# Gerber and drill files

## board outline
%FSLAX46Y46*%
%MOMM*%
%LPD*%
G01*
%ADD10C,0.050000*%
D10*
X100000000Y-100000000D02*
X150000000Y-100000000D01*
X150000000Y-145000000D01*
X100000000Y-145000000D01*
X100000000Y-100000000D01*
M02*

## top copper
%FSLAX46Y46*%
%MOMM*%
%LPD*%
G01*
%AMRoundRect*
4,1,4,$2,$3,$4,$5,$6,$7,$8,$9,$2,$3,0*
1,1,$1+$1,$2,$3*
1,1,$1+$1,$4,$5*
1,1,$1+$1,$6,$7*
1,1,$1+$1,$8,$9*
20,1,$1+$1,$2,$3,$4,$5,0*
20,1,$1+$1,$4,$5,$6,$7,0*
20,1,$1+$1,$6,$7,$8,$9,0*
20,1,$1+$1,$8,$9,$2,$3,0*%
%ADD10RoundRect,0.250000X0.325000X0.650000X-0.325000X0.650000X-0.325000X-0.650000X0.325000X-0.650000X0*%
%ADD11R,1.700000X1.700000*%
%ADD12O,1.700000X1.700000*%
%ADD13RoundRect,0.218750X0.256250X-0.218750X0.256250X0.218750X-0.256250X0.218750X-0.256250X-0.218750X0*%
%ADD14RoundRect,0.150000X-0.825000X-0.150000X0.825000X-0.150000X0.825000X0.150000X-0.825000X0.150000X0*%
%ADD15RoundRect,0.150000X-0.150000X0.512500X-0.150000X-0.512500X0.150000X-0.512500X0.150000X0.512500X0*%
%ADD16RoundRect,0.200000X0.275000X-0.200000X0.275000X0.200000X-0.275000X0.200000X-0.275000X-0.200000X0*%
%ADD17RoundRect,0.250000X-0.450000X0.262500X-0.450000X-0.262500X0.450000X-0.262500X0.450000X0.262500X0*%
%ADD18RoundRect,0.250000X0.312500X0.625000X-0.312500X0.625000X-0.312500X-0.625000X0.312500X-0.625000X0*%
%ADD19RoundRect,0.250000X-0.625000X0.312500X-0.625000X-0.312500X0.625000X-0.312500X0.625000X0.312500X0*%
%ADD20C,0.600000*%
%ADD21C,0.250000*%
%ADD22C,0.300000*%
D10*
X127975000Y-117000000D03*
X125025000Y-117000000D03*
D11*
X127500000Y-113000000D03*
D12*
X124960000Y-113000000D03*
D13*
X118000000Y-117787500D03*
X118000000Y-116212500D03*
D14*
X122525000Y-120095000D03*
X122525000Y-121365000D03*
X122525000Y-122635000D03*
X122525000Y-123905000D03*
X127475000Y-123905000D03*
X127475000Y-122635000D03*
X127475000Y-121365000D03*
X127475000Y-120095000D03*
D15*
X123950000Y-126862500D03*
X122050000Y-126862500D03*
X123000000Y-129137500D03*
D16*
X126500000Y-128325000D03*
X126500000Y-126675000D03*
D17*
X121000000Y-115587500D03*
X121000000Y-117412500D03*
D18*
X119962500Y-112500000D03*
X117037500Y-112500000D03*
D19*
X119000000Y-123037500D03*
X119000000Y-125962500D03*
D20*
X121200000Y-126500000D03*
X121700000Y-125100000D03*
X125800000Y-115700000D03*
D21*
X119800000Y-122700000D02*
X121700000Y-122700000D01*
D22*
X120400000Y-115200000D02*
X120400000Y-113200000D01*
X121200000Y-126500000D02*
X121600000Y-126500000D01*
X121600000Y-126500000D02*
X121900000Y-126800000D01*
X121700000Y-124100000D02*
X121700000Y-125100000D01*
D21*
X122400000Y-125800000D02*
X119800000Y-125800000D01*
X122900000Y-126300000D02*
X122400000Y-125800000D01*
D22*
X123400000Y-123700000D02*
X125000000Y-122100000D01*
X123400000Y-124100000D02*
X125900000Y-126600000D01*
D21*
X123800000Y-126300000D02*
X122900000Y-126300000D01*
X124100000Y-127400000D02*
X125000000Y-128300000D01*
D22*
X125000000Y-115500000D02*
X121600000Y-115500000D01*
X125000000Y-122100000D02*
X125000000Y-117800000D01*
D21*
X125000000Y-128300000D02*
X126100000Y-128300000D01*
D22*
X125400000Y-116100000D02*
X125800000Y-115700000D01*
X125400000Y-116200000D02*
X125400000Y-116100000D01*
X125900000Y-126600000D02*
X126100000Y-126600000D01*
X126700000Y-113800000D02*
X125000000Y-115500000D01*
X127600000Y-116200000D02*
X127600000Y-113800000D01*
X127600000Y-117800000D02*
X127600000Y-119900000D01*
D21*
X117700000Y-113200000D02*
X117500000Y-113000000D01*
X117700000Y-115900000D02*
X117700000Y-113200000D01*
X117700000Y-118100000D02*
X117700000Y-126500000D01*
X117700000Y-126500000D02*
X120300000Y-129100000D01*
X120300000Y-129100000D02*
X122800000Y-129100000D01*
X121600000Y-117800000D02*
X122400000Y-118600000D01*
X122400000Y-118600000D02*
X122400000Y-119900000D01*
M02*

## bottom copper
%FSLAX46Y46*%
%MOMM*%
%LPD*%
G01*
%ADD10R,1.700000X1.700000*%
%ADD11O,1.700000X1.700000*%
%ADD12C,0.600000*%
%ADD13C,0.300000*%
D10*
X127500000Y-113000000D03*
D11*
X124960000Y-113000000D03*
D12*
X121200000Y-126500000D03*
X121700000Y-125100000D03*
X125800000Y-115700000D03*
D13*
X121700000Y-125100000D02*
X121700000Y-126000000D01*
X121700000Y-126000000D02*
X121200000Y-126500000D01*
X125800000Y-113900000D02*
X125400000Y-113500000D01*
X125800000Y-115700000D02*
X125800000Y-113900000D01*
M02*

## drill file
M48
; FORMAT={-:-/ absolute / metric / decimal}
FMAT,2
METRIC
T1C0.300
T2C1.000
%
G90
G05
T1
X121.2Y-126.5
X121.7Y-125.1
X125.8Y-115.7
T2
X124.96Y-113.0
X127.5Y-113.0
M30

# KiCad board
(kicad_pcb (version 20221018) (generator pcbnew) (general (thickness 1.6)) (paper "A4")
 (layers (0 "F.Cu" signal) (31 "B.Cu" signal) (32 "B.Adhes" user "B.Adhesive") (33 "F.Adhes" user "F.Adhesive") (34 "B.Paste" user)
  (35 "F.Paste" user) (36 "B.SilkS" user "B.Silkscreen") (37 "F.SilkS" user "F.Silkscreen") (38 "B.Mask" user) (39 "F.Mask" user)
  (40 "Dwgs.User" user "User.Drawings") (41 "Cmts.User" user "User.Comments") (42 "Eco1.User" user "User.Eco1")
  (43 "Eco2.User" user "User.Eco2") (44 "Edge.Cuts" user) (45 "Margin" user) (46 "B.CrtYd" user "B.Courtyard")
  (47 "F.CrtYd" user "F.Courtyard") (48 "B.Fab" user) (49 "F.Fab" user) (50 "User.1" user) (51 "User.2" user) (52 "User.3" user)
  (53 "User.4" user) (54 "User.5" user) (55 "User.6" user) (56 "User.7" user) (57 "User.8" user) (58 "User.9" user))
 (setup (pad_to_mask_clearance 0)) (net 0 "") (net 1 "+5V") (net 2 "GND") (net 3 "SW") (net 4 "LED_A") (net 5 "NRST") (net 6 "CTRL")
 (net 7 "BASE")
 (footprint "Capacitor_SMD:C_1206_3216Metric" (layer "F.Cu") (at 126.5 117 180)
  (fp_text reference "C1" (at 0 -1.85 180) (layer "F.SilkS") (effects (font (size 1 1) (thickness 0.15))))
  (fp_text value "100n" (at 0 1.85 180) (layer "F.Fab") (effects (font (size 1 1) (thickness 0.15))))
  (pad "1" smd roundrect (at -1.475 0 180) (size 1.15 1.8) (layers "F.Cu" "F.Paste" "F.Mask") (roundrect_rratio 0.217391) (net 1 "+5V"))
  (pad "2" smd roundrect (at 1.475 0 180) (size 1.15 1.8) (layers "F.Cu" "F.Paste" "F.Mask") (roundrect_rratio 0.217391) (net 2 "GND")))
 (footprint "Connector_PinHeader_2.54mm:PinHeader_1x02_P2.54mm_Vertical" (layer "F.Cu") (at 127.5 113 -90)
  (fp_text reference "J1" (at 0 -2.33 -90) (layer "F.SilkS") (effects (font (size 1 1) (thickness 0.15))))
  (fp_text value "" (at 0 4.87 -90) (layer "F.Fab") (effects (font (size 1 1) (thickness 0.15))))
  (pad "1" thru_hole rect (at 0 0 270) (size 1.7 1.7) (drill 1) (layers "*.Cu" "*.Mask") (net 1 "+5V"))
  (pad "2" thru_hole oval (at 0 2.54 270) (size 1.7 1.7) (drill 1) (layers "*.Cu" "*.Mask") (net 2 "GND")))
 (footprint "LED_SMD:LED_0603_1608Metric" (layer "F.Cu") (at 118 117 90)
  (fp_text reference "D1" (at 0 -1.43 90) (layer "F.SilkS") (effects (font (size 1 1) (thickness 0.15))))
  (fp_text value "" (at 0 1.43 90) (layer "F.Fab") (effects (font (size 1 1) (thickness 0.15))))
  (pad "1" smd roundrect (at -0.7875 0 90) (size 0.875 0.95) (layers "F.Cu" "F.Paste" "F.Mask") (roundrect_rratio 0.25) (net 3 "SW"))
  (pad "2" smd roundrect (at 0.7875 0 90) (size 0.875 0.95) (layers "F.Cu" "F.Paste" "F.Mask") (roundrect_rratio 0.25) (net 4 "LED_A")))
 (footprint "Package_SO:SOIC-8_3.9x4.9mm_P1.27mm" (layer "F.Cu") (at 125 122)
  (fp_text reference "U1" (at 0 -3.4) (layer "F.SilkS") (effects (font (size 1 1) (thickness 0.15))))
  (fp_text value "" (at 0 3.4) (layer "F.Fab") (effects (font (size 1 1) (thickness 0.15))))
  (pad "1" smd roundrect (at -2.475 -1.905) (size 1.95 0.6) (layers "F.Cu" "F.Paste" "F.Mask") (roundrect_rratio 0.25) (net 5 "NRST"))
  (pad "2" smd roundrect (at -2.475 -0.635) (size 1.95 0.6) (layers "F.Cu" "F.Paste" "F.Mask") (roundrect_rratio 0.25))
  (pad "3" smd roundrect (at -2.475 0.635) (size 1.95 0.6) (layers "F.Cu" "F.Paste" "F.Mask") (roundrect_rratio 0.25) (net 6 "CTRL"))
  (pad "4" smd roundrect (at -2.475 1.905) (size 1.95 0.6) (layers "F.Cu" "F.Paste" "F.Mask") (roundrect_rratio 0.25) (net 2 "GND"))
  (pad "5" smd roundrect (at 2.475 1.905) (size 1.95 0.6) (layers "F.Cu" "F.Paste" "F.Mask") (roundrect_rratio 0.25))
  (pad "6" smd roundrect (at 2.475 0.635) (size 1.95 0.6) (layers "F.Cu" "F.Paste" "F.Mask") (roundrect_rratio 0.25))
  (pad "7" smd roundrect (at 2.475 -0.635) (size 1.95 0.6) (layers "F.Cu" "F.Paste" "F.Mask") (roundrect_rratio 0.25))
  (pad "8" smd roundrect (at 2.475 -1.905) (size 1.95 0.6) (layers "F.Cu" "F.Paste" "F.Mask") (roundrect_rratio 0.25) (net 1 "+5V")))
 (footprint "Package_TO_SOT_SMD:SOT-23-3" (layer "F.Cu") (at 123 128 -90)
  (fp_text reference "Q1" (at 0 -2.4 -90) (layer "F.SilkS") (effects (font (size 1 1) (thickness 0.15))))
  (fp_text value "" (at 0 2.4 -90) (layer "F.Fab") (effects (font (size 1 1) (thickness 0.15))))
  (pad "1" smd roundrect (at -1.1375 -0.95 270) (size 1.325 0.6) (layers "F.Cu" "F.Paste" "F.Mask") (roundrect_rratio 0.25) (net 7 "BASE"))
  (pad "2" smd roundrect (at -1.1375 0.95 270) (size 1.325 0.6) (layers "F.Cu" "F.Paste" "F.Mask") (roundrect_rratio 0.25) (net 2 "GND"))
  (pad "3" smd roundrect (at 1.1375 0 270) (size 1.325 0.6) (layers "F.Cu" "F.Paste" "F.Mask") (roundrect_rratio 0.25) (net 3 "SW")))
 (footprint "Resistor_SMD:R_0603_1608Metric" (layer "F.Cu") (at 126.5 127.5 90)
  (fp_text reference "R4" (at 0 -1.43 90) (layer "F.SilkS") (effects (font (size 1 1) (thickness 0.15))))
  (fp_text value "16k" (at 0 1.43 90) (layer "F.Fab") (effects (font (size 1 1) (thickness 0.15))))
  (pad "1" smd roundrect (at -0.825 0 90) (size 0.8 0.95) (layers "F.Cu" "F.Paste" "F.Mask") (roundrect_rratio 0.25) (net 7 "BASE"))
  (pad "2" smd roundrect (at 0.825 0 90) (size 0.8 0.95) (layers "F.Cu" "F.Paste" "F.Mask") (roundrect_rratio 0.25) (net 2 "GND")))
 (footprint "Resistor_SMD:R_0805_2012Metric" (layer "F.Cu") (at 121 116.5 -90)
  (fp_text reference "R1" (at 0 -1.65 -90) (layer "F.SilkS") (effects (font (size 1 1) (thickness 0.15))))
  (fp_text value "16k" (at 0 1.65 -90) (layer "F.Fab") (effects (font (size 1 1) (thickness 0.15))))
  (pad "1" smd roundrect (at -0.9125 0 270) (size 1.025 1.4) (layers "F.Cu" "F.Paste" "F.Mask") (roundrect_rratio 0.243902) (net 1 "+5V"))
  (pad "2" smd roundrect (at 0.9125 0 270) (size 1.025 1.4) (layers "F.Cu" "F.Paste" "F.Mask") (roundrect_rratio 0.243902) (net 5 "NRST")))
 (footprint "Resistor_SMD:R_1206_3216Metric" (layer "F.Cu") (at 118.5 112.5 180)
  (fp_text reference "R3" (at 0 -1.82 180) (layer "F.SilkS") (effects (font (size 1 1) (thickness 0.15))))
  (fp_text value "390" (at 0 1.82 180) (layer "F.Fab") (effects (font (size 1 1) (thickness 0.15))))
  (pad "1" smd roundrect (at -1.4625 0 180) (size 1.125 1.75) (layers "F.Cu" "F.Paste" "F.Mask") (roundrect_rratio 0.222222) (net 1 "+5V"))
  (pad "2" smd roundrect (at 1.4625 0 180) (size 1.125 1.75) (layers "F.Cu" "F.Paste" "F.Mask") (roundrect_rratio 0.222222) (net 4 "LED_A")))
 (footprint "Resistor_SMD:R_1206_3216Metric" (layer "F.Cu") (at 119 124.5 -90)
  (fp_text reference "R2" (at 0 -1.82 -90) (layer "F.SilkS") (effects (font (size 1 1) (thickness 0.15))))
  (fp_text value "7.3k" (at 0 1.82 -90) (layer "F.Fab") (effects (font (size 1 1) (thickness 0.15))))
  (pad "1" smd roundrect (at -1.4625 0 270) (size 1.125 1.75) (layers "F.Cu" "F.Paste" "F.Mask") (roundrect_rratio 0.222222) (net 6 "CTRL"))
  (pad "2" smd roundrect (at 1.4625 0 270) (size 1.125 1.75) (layers "F.Cu" "F.Paste" "F.Mask") (roundrect_rratio 0.222222) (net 7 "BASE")))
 (gr_rect (start 100 100) (end 150 145) (stroke (width 0.05) (type default)) (fill none) (layer "Edge.Cuts"))
 (segment (start 119.8 122.7) (end 121.7 122.7) (width 0.25) (layer "F.Cu") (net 6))
 (segment (start 120.4 115.2) (end 120.4 113.2) (width 0.3) (layer "F.Cu") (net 1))
 (segment (start 121.2 126.5) (end 121.6 126.5) (width 0.3) (layer "F.Cu") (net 2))
 (segment (start 121.6 126.5) (end 121.9 126.8) (width 0.3) (layer "F.Cu") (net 2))
 (segment (start 121.7 124.1) (end 121.7 125.1) (width 0.3) (layer "F.Cu") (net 2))
 (segment (start 122.4 125.8) (end 119.8 125.8) (width 0.25) (layer "F.Cu") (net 7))
 (segment (start 122.9 126.3) (end 122.4 125.8) (width 0.25) (layer "F.Cu") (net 7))
 (segment (start 123.4 123.7) (end 125 122.1) (width 0.3) (layer "F.Cu") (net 2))
 (segment (start 123.4 124.1) (end 125.9 126.6) (width 0.3) (layer "F.Cu") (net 2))
 (segment (start 123.8 126.3) (end 122.9 126.3) (width 0.25) (layer "F.Cu") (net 7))
 (segment (start 124.1 127.4) (end 125 128.3) (width 0.25) (layer "F.Cu") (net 7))
 (segment (start 125 115.5) (end 121.6 115.5) (width 0.3) (layer "F.Cu") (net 1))
 (segment (start 125 122.1) (end 125 117.8) (width 0.3) (layer "F.Cu") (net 2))
 (segment (start 125 128.3) (end 126.1 128.3) (width 0.25) (layer "F.Cu") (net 7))
 (segment (start 125.4 116.1) (end 125.8 115.7) (width 0.3) (layer "F.Cu") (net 2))
 (segment (start 125.4 116.2) (end 125.4 116.1) (width 0.3) (layer "F.Cu") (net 2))
 (segment (start 125.9 126.6) (end 126.1 126.6) (width 0.3) (layer "F.Cu") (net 2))
 (segment (start 126.7 113.8) (end 125 115.5) (width 0.3) (layer "F.Cu") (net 1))
 (segment (start 127.6 116.2) (end 127.6 113.8) (width 0.3) (layer "F.Cu") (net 1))
 (segment (start 127.6 117.8) (end 127.6 119.9) (width 0.3) (layer "F.Cu") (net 1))
 (via (at 121.2 126.5) (size 0.6) (drill 0.3) (layers "F.Cu" "B.Cu") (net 2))
 (via (at 121.7 125.1) (size 0.6) (drill 0.3) (layers "F.Cu" "B.Cu") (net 2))
 (via (at 125.8 115.7) (size 0.6) (drill 0.3) (layers "F.Cu" "B.Cu") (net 2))
 (segment (start 117.7 113.2) (end 117.5 113) (width 0.25) (layer "F.Cu") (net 4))
 (segment (start 117.7 115.9) (end 117.7 113.2) (width 0.25) (layer "F.Cu") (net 4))
 (segment (start 117.7 118.1) (end 117.7 126.5) (width 0.25) (layer "F.Cu") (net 3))
 (segment (start 117.7 126.5) (end 120.3 129.1) (width 0.25) (layer "F.Cu") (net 3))
 (segment (start 120.3 129.1) (end 122.8 129.1) (width 0.25) (layer "F.Cu") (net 3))
 (segment (start 121.6 117.8) (end 122.4 118.6) (width 0.25) (layer "F.Cu") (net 5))
 (segment (start 121.7 125.1) (end 121.7 126) (width 0.3) (layer "B.Cu") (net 2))
 (segment (start 121.7 126) (end 121.2 126.5) (width 0.3) (layer "B.Cu") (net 2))
 (segment (start 122.4 118.6) (end 122.4 119.9) (width 0.25) (layer "F.Cu") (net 5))
 (segment (start 125.8 113.9) (end 125.4 113.5) (width 0.3) (layer "B.Cu") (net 2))
 (segment (start 125.8 115.7) (end 125.8 113.9) (width 0.3) (layer "B.Cu") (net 2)))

